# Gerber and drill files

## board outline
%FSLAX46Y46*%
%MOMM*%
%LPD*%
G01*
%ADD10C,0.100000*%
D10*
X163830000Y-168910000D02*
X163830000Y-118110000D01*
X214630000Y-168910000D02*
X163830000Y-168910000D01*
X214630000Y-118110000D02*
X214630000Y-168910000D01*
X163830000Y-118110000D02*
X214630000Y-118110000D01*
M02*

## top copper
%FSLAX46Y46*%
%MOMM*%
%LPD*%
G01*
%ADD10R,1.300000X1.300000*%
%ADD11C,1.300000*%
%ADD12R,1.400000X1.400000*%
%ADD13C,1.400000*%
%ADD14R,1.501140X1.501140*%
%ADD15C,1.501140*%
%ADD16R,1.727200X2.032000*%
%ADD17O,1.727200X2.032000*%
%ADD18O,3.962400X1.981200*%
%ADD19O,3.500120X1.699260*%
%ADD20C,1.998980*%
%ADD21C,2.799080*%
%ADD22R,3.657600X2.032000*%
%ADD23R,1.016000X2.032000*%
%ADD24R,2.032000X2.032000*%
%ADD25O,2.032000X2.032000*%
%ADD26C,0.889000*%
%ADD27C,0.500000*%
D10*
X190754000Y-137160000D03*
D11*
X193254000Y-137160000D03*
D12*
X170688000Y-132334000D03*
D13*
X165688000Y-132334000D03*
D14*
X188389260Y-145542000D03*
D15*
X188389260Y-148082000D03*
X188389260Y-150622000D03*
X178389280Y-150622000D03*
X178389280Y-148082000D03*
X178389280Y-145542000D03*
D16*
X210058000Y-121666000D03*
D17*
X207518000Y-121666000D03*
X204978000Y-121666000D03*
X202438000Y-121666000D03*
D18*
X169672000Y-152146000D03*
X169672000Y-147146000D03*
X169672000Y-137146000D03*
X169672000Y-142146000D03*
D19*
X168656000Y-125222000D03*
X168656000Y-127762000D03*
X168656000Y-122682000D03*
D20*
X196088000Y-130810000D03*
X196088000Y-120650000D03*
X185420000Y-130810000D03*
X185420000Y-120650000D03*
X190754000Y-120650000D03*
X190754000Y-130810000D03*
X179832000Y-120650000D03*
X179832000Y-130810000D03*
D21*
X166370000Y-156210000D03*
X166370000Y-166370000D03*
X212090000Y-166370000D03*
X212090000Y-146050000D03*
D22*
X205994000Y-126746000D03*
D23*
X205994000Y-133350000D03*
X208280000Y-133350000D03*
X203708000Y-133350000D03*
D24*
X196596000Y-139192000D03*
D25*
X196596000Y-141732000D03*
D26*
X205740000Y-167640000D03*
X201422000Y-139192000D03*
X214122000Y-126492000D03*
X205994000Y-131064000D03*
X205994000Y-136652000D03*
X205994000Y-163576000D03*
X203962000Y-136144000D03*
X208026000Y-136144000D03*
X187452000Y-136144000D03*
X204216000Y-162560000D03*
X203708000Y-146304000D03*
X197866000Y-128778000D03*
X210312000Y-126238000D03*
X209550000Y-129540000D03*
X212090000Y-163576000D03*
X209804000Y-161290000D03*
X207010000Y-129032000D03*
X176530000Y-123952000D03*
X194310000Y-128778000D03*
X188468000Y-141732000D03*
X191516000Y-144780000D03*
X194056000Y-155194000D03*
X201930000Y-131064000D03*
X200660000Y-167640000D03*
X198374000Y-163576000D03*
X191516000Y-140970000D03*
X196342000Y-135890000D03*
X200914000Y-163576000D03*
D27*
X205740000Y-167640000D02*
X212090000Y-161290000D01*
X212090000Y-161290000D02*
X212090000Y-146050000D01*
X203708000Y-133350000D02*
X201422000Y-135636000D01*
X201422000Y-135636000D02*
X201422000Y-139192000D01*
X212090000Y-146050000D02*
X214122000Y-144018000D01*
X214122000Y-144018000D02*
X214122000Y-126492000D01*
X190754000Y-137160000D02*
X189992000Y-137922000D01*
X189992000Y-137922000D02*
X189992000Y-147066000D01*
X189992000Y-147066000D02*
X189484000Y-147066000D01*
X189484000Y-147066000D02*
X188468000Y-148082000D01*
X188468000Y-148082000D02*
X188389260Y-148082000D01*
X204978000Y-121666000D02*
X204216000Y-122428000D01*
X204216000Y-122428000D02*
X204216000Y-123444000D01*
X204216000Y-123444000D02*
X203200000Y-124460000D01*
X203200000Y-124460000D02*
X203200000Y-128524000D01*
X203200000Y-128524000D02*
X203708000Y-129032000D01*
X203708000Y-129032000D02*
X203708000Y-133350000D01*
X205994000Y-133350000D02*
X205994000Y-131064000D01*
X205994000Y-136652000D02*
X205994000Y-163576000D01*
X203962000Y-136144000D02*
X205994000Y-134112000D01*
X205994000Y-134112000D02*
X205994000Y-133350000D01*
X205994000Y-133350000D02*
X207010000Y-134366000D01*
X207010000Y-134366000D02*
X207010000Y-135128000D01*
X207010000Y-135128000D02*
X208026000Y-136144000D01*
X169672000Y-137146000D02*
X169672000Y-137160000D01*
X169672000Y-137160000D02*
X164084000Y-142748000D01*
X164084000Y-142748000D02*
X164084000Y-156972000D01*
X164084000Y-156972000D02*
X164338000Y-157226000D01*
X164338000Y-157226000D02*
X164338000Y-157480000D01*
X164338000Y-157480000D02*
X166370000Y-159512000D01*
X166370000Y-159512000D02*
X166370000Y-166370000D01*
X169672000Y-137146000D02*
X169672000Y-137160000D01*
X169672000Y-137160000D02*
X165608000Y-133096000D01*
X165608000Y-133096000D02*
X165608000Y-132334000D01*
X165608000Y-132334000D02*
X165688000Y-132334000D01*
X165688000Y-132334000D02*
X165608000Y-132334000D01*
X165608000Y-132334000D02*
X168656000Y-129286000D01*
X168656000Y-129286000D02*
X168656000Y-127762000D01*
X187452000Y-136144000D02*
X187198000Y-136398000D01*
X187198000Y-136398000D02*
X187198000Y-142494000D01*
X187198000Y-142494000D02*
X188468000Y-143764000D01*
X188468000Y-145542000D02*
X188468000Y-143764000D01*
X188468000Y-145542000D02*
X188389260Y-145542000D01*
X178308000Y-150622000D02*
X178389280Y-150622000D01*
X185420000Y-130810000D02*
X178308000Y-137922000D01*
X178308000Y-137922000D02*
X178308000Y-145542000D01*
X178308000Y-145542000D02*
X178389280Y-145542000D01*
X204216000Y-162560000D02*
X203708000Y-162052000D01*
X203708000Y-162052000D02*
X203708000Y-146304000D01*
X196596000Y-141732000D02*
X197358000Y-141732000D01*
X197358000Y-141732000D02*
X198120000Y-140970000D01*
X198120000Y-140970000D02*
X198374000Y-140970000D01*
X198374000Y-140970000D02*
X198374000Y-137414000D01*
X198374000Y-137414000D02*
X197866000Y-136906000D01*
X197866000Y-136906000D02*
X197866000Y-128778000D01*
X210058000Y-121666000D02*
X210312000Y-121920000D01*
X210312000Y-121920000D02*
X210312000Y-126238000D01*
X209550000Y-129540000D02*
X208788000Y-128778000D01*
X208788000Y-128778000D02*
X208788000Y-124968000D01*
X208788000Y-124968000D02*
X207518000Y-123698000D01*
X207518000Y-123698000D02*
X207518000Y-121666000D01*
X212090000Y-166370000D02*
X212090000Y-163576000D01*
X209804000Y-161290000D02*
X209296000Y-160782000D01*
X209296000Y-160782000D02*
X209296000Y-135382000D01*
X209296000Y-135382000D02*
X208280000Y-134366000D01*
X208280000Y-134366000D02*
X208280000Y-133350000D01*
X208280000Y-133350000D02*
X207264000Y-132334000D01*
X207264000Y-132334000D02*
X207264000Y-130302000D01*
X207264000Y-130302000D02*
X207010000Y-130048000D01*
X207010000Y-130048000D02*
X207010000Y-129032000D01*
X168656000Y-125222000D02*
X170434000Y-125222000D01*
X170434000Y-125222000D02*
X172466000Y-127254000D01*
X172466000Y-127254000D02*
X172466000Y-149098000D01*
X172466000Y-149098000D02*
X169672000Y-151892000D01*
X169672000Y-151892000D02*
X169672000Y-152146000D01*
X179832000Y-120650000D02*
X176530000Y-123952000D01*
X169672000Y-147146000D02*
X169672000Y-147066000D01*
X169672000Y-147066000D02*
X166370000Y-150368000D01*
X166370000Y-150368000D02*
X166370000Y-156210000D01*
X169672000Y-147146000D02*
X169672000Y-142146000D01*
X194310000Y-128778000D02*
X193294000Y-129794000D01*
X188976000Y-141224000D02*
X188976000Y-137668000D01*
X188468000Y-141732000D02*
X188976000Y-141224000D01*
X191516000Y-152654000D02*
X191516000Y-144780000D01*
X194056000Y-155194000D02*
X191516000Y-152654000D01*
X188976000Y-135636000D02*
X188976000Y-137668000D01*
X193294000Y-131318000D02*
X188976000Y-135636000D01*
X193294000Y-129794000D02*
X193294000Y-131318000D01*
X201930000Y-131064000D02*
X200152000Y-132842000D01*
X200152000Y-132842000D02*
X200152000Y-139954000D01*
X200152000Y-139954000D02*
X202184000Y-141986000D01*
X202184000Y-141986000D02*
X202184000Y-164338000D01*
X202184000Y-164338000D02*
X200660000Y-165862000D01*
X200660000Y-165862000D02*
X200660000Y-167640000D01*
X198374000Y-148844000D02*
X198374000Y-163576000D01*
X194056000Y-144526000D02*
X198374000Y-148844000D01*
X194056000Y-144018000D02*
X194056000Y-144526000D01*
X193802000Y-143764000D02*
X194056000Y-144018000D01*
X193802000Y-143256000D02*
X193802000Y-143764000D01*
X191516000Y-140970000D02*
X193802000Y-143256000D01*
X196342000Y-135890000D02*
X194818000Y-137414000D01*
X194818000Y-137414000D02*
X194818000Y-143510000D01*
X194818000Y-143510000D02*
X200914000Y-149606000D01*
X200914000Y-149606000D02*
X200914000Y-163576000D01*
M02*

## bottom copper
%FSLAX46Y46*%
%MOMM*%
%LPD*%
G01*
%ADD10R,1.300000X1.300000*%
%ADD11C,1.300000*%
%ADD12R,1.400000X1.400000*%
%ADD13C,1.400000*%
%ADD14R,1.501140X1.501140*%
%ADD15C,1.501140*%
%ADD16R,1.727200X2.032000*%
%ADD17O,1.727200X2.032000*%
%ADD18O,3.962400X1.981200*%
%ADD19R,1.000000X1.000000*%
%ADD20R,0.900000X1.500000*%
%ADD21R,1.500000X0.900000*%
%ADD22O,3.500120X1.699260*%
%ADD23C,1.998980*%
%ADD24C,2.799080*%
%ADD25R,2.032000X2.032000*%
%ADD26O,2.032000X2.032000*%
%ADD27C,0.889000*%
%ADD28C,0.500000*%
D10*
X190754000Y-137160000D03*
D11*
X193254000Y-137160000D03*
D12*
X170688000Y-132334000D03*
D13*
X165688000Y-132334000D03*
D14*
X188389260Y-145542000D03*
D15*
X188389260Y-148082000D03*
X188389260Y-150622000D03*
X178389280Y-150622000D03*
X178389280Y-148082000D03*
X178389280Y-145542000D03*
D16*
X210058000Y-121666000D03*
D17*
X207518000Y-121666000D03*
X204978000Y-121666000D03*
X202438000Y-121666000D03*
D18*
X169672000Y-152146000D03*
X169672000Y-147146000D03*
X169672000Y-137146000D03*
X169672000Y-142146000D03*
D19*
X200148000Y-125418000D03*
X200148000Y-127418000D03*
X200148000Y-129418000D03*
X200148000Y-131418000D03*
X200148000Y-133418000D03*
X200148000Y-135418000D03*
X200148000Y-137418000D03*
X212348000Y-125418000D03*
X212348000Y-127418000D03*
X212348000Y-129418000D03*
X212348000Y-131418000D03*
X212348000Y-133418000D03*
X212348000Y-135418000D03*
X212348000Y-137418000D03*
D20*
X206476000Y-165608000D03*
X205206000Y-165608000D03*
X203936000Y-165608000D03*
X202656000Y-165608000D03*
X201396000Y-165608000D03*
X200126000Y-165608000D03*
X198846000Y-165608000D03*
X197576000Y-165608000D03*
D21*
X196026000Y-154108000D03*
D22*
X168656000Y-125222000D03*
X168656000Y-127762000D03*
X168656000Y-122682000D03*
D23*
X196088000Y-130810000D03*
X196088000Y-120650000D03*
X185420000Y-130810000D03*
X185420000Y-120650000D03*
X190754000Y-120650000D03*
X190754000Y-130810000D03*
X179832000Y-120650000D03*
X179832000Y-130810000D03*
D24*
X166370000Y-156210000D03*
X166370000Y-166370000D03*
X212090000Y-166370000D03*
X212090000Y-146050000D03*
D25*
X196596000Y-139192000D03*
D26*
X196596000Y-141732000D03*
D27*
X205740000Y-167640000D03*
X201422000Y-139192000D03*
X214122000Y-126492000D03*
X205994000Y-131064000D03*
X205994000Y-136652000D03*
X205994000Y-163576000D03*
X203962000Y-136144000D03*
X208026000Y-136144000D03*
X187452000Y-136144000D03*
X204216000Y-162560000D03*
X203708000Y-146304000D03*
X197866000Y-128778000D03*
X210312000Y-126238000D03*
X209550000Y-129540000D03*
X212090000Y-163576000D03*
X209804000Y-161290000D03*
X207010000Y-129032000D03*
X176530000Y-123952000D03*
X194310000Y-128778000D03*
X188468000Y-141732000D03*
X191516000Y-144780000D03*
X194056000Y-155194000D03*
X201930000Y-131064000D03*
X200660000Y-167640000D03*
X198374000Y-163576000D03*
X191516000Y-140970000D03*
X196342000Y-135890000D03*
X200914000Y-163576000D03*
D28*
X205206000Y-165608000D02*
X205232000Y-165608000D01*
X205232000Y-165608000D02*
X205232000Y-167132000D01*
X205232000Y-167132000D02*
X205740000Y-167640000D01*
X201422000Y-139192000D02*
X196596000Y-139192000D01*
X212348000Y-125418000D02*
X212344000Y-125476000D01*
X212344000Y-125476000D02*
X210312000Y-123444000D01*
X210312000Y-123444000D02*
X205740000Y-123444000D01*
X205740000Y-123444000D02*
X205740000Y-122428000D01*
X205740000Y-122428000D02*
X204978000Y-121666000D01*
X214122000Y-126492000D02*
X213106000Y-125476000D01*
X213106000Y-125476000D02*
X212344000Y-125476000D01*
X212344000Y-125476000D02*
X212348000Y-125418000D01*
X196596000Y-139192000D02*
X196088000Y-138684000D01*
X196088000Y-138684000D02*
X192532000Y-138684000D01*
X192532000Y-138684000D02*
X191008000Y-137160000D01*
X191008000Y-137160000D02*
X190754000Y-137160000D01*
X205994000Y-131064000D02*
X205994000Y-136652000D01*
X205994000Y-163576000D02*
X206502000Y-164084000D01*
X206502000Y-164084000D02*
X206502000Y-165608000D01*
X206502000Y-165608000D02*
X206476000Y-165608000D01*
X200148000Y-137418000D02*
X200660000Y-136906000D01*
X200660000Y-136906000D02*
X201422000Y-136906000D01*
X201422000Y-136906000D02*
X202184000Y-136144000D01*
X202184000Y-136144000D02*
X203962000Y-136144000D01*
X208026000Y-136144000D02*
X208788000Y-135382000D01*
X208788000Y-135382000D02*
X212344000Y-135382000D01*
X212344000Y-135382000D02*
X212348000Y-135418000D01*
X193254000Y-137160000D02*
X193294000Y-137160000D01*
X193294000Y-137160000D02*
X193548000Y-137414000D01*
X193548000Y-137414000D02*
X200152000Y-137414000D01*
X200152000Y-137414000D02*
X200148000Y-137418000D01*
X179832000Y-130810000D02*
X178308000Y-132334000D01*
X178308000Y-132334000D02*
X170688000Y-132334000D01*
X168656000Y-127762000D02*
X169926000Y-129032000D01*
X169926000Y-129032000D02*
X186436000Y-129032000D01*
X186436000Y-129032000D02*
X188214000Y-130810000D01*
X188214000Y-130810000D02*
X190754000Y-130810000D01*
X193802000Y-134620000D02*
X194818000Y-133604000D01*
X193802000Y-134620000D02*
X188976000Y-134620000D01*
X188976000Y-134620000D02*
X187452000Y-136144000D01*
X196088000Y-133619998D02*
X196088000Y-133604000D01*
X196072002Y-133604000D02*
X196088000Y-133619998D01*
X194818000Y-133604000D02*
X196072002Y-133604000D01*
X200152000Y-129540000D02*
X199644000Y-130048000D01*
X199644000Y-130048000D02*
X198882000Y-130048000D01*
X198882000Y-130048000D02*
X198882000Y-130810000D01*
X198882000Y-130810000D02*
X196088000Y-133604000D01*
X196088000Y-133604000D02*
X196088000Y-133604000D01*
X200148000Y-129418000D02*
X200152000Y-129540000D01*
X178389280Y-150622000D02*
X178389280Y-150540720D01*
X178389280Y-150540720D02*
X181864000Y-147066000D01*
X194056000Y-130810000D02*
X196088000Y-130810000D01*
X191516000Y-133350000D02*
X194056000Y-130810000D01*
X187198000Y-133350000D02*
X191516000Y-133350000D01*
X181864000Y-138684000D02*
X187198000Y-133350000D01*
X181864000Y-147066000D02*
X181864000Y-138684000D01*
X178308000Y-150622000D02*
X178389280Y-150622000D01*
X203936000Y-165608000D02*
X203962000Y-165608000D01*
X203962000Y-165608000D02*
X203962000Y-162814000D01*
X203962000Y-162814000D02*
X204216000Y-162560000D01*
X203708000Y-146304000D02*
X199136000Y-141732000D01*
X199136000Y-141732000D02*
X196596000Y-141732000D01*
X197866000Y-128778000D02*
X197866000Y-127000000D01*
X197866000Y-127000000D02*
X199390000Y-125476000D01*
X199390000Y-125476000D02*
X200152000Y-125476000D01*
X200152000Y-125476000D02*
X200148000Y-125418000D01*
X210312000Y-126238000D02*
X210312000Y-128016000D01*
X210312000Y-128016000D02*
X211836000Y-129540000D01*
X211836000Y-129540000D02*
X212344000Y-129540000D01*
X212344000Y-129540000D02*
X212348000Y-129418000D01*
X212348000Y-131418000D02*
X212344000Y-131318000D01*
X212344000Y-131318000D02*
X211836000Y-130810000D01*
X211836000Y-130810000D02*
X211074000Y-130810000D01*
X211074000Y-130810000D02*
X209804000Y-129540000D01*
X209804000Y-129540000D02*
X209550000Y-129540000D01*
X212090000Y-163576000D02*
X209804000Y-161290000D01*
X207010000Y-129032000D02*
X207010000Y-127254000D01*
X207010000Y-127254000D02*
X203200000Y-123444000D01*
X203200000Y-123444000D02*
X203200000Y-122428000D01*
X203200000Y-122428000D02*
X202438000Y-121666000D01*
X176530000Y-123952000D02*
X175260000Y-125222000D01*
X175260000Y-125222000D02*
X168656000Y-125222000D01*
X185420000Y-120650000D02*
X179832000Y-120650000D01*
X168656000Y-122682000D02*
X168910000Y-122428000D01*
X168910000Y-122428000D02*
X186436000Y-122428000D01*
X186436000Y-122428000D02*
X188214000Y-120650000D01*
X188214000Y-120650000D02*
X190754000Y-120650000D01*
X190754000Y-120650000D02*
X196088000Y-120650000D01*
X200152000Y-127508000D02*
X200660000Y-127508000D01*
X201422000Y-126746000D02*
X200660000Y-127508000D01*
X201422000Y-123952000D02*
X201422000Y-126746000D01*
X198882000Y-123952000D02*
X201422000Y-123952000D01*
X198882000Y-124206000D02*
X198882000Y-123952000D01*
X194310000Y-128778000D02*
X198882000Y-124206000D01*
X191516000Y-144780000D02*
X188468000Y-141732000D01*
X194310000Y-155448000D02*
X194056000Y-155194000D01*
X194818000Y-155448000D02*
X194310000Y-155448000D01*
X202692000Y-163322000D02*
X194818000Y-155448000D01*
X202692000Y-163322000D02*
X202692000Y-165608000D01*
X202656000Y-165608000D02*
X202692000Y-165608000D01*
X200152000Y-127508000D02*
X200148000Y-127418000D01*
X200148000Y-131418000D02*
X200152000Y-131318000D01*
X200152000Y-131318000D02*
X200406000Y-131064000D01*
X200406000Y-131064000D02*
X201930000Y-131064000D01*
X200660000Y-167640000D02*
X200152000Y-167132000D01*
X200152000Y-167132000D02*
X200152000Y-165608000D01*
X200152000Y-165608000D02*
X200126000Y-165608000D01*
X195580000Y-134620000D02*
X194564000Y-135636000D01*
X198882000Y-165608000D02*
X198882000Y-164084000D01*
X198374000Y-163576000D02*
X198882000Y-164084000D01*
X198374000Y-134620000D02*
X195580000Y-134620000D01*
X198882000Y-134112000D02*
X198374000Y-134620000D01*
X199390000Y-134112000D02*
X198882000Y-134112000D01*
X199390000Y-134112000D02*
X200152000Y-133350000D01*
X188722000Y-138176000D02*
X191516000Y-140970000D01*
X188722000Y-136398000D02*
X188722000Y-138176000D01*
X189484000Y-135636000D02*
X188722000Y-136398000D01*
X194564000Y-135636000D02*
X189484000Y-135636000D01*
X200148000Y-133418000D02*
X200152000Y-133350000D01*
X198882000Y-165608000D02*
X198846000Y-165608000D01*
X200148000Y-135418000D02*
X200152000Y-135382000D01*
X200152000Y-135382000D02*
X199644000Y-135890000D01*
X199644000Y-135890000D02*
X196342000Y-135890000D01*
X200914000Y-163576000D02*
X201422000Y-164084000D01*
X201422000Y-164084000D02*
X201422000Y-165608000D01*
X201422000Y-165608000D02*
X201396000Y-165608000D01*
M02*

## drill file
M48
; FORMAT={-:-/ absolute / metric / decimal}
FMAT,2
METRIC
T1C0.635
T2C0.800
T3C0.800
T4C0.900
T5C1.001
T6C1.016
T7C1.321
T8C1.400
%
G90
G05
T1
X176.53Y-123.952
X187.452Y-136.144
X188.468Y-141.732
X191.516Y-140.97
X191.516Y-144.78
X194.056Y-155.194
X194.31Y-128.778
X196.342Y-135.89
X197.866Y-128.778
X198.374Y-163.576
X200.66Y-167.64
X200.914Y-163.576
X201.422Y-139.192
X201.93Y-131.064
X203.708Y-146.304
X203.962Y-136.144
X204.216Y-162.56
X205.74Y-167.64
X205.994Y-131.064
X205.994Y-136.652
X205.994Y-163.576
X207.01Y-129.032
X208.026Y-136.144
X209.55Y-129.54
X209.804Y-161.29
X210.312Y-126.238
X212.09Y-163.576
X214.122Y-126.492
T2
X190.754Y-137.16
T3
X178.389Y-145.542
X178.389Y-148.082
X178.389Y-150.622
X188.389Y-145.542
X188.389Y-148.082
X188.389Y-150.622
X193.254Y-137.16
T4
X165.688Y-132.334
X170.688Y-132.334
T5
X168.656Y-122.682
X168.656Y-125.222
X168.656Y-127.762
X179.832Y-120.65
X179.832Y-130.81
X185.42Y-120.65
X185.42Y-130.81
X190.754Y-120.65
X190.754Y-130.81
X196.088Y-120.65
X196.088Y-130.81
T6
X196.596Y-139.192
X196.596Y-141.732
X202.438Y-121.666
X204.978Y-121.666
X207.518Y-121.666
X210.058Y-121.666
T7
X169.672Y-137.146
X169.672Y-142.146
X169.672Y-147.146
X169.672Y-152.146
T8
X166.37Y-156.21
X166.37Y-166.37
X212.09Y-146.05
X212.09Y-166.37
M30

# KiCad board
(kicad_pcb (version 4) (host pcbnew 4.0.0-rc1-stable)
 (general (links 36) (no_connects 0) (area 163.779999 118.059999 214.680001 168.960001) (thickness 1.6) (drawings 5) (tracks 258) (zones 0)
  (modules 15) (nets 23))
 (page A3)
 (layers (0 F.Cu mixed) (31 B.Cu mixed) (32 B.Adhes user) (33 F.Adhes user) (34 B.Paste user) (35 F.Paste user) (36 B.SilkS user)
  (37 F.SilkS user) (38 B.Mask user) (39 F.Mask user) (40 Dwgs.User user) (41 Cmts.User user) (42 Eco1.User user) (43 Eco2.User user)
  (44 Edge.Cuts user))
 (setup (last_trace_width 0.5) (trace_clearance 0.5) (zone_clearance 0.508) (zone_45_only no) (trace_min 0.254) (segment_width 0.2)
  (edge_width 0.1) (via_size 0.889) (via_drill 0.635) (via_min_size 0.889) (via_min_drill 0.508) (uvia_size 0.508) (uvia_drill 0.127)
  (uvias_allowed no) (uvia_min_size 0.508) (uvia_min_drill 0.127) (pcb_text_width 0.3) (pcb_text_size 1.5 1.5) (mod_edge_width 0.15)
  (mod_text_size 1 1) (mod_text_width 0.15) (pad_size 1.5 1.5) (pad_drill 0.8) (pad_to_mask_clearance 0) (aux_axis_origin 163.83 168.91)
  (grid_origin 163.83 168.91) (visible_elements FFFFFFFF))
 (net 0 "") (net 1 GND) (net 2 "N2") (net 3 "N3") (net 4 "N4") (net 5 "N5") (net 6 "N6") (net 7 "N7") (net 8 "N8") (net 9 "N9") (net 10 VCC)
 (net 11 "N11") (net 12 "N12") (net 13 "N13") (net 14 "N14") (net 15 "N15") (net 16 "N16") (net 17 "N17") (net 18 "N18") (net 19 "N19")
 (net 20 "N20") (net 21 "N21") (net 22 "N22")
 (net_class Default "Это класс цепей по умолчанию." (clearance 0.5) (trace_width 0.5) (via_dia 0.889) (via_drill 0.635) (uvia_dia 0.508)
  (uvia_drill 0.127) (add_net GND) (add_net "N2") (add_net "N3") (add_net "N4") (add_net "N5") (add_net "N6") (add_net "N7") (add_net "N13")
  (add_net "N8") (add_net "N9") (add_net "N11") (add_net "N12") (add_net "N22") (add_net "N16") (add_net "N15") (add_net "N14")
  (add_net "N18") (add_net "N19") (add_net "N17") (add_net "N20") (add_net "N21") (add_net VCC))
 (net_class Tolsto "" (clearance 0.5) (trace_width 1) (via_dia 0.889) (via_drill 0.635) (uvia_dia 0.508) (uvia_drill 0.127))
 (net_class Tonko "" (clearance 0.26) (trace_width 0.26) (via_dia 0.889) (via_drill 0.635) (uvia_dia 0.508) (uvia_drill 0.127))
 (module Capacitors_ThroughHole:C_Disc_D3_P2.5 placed (layer B.Cu) (at 190.754 137.16)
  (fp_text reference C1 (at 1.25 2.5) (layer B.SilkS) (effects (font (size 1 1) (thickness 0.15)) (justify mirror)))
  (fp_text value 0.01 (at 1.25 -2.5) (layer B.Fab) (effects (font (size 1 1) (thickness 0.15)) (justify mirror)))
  (pad 1 thru_hole rect (at 0 0) (size 1.3 1.3) (drill 0.8) (layers *.Cu *.Mask B.SilkS) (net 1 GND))
  (pad 2 thru_hole circle (at 2.5 0) (size 1.3 1.3) (drill 0.8001) (layers *.Cu *.Mask B.SilkS) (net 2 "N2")))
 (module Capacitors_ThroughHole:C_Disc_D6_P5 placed (layer F.Cu) (at 170.688 132.334 180)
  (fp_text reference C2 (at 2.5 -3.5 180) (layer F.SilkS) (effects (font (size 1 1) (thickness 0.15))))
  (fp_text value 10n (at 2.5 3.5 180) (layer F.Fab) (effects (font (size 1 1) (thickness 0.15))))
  (pad 1 thru_hole rect (at 0 0 180) (size 1.4 1.4) (drill 0.9) (layers *.Cu *.Mask F.SilkS) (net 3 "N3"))
  (pad 2 thru_hole circle (at 5 0 180) (size 1.4 1.4) (drill 0.9) (layers *.Cu *.Mask F.SilkS) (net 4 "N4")))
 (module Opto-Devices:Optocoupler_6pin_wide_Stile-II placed (layer B.Cu) (at 183.388 148.082 270)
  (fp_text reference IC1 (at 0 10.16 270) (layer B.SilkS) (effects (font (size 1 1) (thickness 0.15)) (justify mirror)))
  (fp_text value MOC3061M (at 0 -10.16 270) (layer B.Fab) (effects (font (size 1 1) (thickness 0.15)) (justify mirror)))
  (pad 1 thru_hole rect (at -2.54 -5.00126 270) (size 1.50114 1.50114) (drill 0.8001) (layers *.Cu *.Mask B.SilkS) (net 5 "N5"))
  (pad 2 thru_hole circle (at 0 -5.00126 270) (size 1.50114 1.50114) (drill 0.8001) (layers *.Cu *.Mask B.SilkS) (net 1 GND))
  (pad 3 thru_hole circle (at 2.54 -5.00126 270) (size 1.50114 1.50114) (drill 0.8001) (layers *.Cu *.Mask B.SilkS))
  (pad 4 thru_hole circle (at 2.54 4.99872 270) (size 1.50114 1.50114) (drill 0.8001) (layers *.Cu *.Mask B.SilkS) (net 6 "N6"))
  (pad 5 thru_hole circle (at 0 4.99872 270) (size 1.50114 1.50114) (drill 0.8001) (layers *.Cu *.Mask B.SilkS))
  (pad 6 thru_hole circle (at -2.54 4.99872 270) (size 1.50114 1.50114) (drill 0.8001) (layers *.Cu *.Mask B.SilkS) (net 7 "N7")))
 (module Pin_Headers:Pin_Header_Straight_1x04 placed (layer F.Cu) (at 210.058 121.666 270)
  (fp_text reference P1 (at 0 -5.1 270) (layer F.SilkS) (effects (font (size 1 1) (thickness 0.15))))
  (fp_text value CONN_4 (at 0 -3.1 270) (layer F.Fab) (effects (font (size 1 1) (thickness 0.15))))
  (pad 1 thru_hole rect (at 0 0 270) (size 2.032 1.7272) (drill 1.016) (layers *.Cu *.Mask F.SilkS) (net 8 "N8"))
  (pad 2 thru_hole oval (at 0 2.54 270) (size 2.032 1.7272) (drill 1.016) (layers *.Cu *.Mask F.SilkS) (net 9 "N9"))
  (pad 3 thru_hole oval (at 0 5.08 270) (size 2.032 1.7272) (drill 1.016) (layers *.Cu *.Mask F.SilkS) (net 1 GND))
  (pad 4 thru_hole oval (at 0 7.62 270) (size 2.032 1.7272) (drill 1.016) (layers *.Cu *.Mask F.SilkS) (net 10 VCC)))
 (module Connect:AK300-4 (layer B.Cu) (at 169.672 152.146 90)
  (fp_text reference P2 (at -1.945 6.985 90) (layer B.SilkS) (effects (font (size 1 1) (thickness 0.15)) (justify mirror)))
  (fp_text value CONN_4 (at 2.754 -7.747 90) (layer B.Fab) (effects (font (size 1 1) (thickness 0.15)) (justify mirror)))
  (pad 1 thru_hole oval (at 0 0 90) (size 1.9812 3.9624) (drill 1.3208) (layers *.Cu B.Paste B.SilkS B.Mask) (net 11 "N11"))
  (pad 2 thru_hole oval (at 5 0 90) (size 1.9812 3.9624) (drill 1.3208) (layers *.Cu B.Paste B.SilkS B.Mask) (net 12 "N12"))
  (pad 4 thru_hole oval (at 15 0 90) (size 1.9812 3.9624) (drill 1.3208) (layers *.Cu B.Paste B.SilkS B.Mask) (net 4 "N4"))
  (pad 3 thru_hole oval (at 10 0 90) (size 1.9812 3.9624) (drill 1.3208) (layers *.Cu *.Mask B.SilkS) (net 12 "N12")))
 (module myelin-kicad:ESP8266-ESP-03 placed (layer B.Cu) (at 206.248 131.318)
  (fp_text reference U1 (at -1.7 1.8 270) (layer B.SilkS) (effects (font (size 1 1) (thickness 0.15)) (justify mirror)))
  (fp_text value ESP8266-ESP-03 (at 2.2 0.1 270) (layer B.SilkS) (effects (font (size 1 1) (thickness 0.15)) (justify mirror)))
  (pad 14 smd rect (at -6.1 -5.9) (size 1 1) (layers B.Cu B.Paste B.Mask) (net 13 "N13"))
  (pad 13 smd rect (at -6.1 -3.9) (size 1 1) (layers B.Cu B.Paste B.Mask) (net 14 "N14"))
  (pad 12 smd rect (at -6.1 -1.9) (size 1 1) (layers B.Cu B.Paste B.Mask) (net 5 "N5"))
  (pad 11 smd rect (at -6.1 0.1) (size 1 1) (layers B.Cu B.Paste B.Mask) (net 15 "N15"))
  (pad 10 smd rect (at -6.1 2.1) (size 1 1) (layers B.Cu B.Paste B.Mask) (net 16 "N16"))
  (pad 9 smd rect (at -6.1 4.1) (size 1 1) (layers B.Cu B.Paste B.Mask) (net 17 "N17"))
  (pad 8 smd rect (at -6.1 6.1) (size 1 1) (layers B.Cu B.Paste B.Mask) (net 2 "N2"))
  (pad 1 smd rect (at 6.1 -5.9) (size 1 1) (layers B.Cu B.Paste B.Mask) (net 1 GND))
  (pad 2 smd rect (at 6.1 -3.9) (size 1 1) (layers B.Cu B.Paste B.Mask))
  (pad 3 smd rect (at 6.1 -1.9) (size 1 1) (layers B.Cu B.Paste B.Mask) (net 8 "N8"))
  (pad 4 smd rect (at 6.1 0.1) (size 1 1) (layers B.Cu B.Paste B.Mask) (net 9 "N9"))
  (pad 5 smd rect (at 6.1 2.1) (size 1 1) (layers B.Cu B.Paste B.Mask) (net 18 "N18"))
  (pad 6 smd rect (at 6.1 4.1) (size 1 1) (layers B.Cu B.Paste B.Mask) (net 2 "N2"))
  (pad 7 smd rect (at 6.1 6.1) (size 1 1) (layers B.Cu B.Paste B.Mask) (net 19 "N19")))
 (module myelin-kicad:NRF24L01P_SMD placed (layer B.Cu) (at 208.026 165.608 90)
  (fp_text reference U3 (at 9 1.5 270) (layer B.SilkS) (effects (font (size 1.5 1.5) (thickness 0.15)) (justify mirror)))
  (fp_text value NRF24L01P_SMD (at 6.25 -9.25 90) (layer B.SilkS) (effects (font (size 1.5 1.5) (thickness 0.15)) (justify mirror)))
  (pad 1 smd rect (at 0 -1.55 90) (size 1.5 0.9) (layers B.Cu B.Paste B.Mask) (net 2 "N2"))
  (pad 2 smd rect (at 0 -2.82 90) (size 1.5 0.9) (layers B.Cu B.Paste B.Mask) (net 1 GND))
  (pad 3 smd rect (at 0 -4.09 90) (size 1.5 0.9) (layers B.Cu B.Paste B.Mask) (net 13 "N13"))
  (pad 4 smd rect (at 0 -5.37 90) (size 1.5 0.9) (layers B.Cu B.Paste B.Mask) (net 14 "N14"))
  (pad 5 smd rect (at 0 -6.63 90) (size 1.5 0.9) (layers B.Cu B.Paste B.Mask) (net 17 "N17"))
  (pad 6 smd rect (at 0 -7.9 90) (size 1.5 0.9) (layers B.Cu B.Paste B.Mask) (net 15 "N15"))
  (pad 7 smd rect (at 0 -9.18 90) (size 1.5 0.9) (layers B.Cu B.Paste B.Mask) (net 16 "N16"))
  (pad 8 smd rect (at 0 -10.45 90) (size 1.5 0.9) (layers B.Cu B.Paste B.Mask) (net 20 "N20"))
  (pad 9 smd rect (at 11.5 -12 90) (size 0.9 1.5) (layers B.Cu B.Paste B.Mask) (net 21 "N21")))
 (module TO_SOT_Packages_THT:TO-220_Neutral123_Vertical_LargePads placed (layer F.Cu) (at 168.656 125.222 90)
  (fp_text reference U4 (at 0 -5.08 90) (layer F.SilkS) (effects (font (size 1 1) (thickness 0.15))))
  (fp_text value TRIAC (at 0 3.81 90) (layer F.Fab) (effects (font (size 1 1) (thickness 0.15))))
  (pad 2 thru_hole oval (at 0 0 180) (size 3.50012 1.69926) (drill 1.00076) (layers *.Cu *.Mask F.SilkS) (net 11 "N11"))
  (pad 1 thru_hole oval (at -2.54 0 180) (size 3.50012 1.69926) (drill 1.00076) (layers *.Cu *.Mask F.SilkS) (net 4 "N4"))
  (pad 3 thru_hole oval (at 2.54 0 180) (size 3.50012 1.69926) (drill 1.00076) (layers *.Cu *.Mask F.SilkS) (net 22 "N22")))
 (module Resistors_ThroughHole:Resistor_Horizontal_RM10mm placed (layer F.Cu) (at 196.088 125.73 90)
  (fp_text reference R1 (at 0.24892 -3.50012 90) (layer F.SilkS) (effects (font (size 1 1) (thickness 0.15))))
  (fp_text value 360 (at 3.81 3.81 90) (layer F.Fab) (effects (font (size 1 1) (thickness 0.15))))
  (pad 1 thru_hole circle (at -5.08 0 90) (size 1.99898 1.99898) (drill 1.00076) (layers *.Cu *.SilkS *.Mask) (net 6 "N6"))
  (pad 2 thru_hole circle (at 5.08 0 90) (size 1.99898 1.99898) (drill 1.00076) (layers *.Cu *.SilkS *.Mask) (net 22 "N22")))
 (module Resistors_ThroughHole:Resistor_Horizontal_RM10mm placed (layer F.Cu) (at 185.42 125.73 90)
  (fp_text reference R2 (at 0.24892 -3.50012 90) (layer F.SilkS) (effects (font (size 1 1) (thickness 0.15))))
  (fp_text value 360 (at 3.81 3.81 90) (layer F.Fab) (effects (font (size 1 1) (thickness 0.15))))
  (pad 1 thru_hole circle (at -5.08 0 90) (size 1.99898 1.99898) (drill 1.00076) (layers *.Cu *.SilkS *.Mask) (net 7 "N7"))
  (pad 2 thru_hole circle (at 5.08 0 90) (size 1.99898 1.99898) (drill 1.00076) (layers *.Cu *.SilkS *.Mask) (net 11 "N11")))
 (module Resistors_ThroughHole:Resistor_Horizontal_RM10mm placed (layer F.Cu) (at 190.754 125.73 270)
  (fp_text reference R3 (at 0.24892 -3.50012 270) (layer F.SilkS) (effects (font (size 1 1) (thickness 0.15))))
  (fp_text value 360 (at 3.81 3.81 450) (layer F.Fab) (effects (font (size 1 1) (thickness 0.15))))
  (pad 1 thru_hole circle (at -5.08 0 270) (size 1.99898 1.99898) (drill 1.00076) (layers *.Cu *.SilkS *.Mask) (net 22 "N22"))
  (pad 2 thru_hole circle (at 5.08 0 270) (size 1.99898 1.99898) (drill 1.00076) (layers *.Cu *.SilkS *.Mask) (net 4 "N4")))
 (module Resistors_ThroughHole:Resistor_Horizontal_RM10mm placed (layer F.Cu) (at 179.832 125.73 270)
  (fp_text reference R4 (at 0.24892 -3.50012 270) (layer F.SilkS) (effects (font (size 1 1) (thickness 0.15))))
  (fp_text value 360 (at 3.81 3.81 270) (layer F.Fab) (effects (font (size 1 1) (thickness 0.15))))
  (pad 1 thru_hole circle (at -5.08 0 270) (size 1.99898 1.99898) (drill 1.00076) (layers *.Cu *.SilkS *.Mask) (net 11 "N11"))
  (pad 2 thru_hole circle (at 5.08 0 270) (size 1.99898 1.99898) (drill 1.00076) (layers *.Cu *.SilkS *.Mask) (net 3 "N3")))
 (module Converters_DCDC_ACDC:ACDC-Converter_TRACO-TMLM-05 (layer F.Cu) (at 166.37 156.21)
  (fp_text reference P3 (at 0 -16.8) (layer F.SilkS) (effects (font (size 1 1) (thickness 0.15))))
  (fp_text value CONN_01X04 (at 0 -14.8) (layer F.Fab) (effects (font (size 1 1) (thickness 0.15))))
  (pad 1 thru_hole circle (at 0 0) (size 2.79908 2.79908) (drill 1.39954) (layers *.Cu *.Mask F.SilkS) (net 12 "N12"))
  (pad 2 thru_hole circle (at 0 10.16) (size 2.79908 2.79908) (drill 1.39954) (layers *.Cu *.Mask F.SilkS) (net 4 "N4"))
  (pad 3 thru_hole circle (at 45.72 10.16) (size 2.79908 2.79908) (drill 1.39954) (layers *.Cu *.Mask F.SilkS) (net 10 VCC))
  (pad 4 thru_hole circle (at 45.72 -10.16) (size 2.79908 2.79908) (drill 1.39954) (layers *.Cu *.Mask F.SilkS) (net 1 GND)))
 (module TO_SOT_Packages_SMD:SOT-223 (layer F.Cu) (at 205.994 130.048)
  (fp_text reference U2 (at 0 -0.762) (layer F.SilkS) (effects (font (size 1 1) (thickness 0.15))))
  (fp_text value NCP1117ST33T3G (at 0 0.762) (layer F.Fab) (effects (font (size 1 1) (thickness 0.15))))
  (pad 4 smd rect (at 0 -3.302) (size 3.6576 2.032) (layers F.Cu F.Paste F.Mask))
  (pad 2 smd rect (at 0 3.302) (size 1.016 2.032) (layers F.Cu F.Paste F.Mask) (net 2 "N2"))
  (pad 3 smd rect (at 2.286 3.302) (size 1.016 2.032) (layers F.Cu F.Paste F.Mask) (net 10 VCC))
  (pad 1 smd rect (at -2.286 3.302) (size 1.016 2.032) (layers F.Cu F.Paste F.Mask) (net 1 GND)))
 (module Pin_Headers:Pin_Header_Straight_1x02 (layer F.Cu) (at 196.596 139.192)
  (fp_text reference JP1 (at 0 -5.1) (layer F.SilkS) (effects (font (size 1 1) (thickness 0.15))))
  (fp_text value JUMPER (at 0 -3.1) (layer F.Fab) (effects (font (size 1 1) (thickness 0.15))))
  (pad 1 thru_hole rect (at 0 0) (size 2.032 2.032) (drill 1.016) (layers *.Cu *.Mask F.SilkS) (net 1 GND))
  (pad 2 thru_hole oval (at 0 2.54) (size 2.032 2.032) (drill 1.016) (layers *.Cu *.Mask F.SilkS) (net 13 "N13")))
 (gr_line (start 163.83 168.91) (end 163.83 118.11) (angle 90) (layer Edge.Cuts) (width 0.1))
 (gr_line (start 214.63 168.91) (end 163.83 168.91) (angle 90) (layer Edge.Cuts) (width 0.1))
 (gr_line (start 214.63 118.11) (end 214.63 168.91) (angle 90) (layer Edge.Cuts) (width 0.1))
 (gr_line (start 163.83 118.11) (end 214.63 118.11) (angle 90) (layer Edge.Cuts) (width 0.1))
 (segment (start 205.206 165.608) (end 205.232 165.608) (width 0.5) (layer B.Cu) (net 1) (status 80000))
 (segment (start 205.232 165.608) (end 205.232 167.132) (width 0.5) (layer B.Cu) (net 1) (status 80000))
 (segment (start 205.232 167.132) (end 205.74 167.64) (width 0.5) (layer B.Cu) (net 1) (status 80000))
 (via (at 205.74 167.64) (size 0.889) (layers F.Cu B.Cu) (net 1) (status 80000))
 (segment (start 205.74 167.64) (end 212.09 161.29) (width 0.5) (layer F.Cu) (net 1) (status 80000))
 (segment (start 212.09 161.29) (end 212.09 146.05) (width 0.5) (layer F.Cu) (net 1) (status 80000))
 (segment (start 203.708 133.35) (end 201.422 135.636) (width 0.5) (layer F.Cu) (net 1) (status 80000))
 (segment (start 201.422 135.636) (end 201.422 139.192) (width 0.5) (layer F.Cu) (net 1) (status 80000))
 (via (at 201.422 139.192) (size 0.889) (layers F.Cu B.Cu) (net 1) (status 80000))
 (segment (start 201.422 139.192) (end 196.596 139.192) (width 0.5) (layer B.Cu) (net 1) (status 80000))
 (segment (start 212.348 125.418) (end 212.344 125.476) (width 0.5) (layer B.Cu) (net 1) (status 80000))
 (segment (start 212.344 125.476) (end 210.312 123.444) (width 0.5) (layer B.Cu) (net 1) (status 80000))
 (segment (start 210.312 123.444) (end 205.74 123.444) (width 0.5) (layer B.Cu) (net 1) (status 80000))
 (segment (start 205.74 123.444) (end 205.74 122.428) (width 0.5) (layer B.Cu) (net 1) (status 80000))
 (segment (start 205.74 122.428) (end 204.978 121.666) (width 0.5) (layer B.Cu) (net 1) (status 80000))
 (segment (start 212.09 146.05) (end 214.122 144.018) (width 0.5) (layer F.Cu) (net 1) (status 80000))
 (segment (start 214.122 144.018) (end 214.122 126.492) (width 0.5) (layer F.Cu) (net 1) (status 80000))
 (via (at 214.122 126.492) (size 0.889) (layers F.Cu B.Cu) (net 1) (status 80000))
 (segment (start 214.122 126.492) (end 213.106 125.476) (width 0.5) (layer B.Cu) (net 1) (status 80000))
 (segment (start 213.106 125.476) (end 212.344 125.476) (width 0.5) (layer B.Cu) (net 1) (status 80000))
 (segment (start 212.344 125.476) (end 212.348 125.418) (width 0.5) (layer B.Cu) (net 1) (status 80000))
 (segment (start 190.754 137.16) (end 189.992 137.922) (width 0.5) (layer F.Cu) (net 1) (status 80000))
 (segment (start 189.992 137.922) (end 189.992 147.066) (width 0.5) (layer F.Cu) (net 1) (status 80000))
 (segment (start 189.992 147.066) (end 189.484 147.066) (width 0.5) (layer F.Cu) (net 1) (status 80000))
 (segment (start 189.484 147.066) (end 188.468 148.082) (width 0.5) (layer F.Cu) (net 1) (status 80000))
 (segment (start 188.468 148.082) (end 188.38926 148.082) (width 0.5) (layer F.Cu) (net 1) (status 80000))
 (segment (start 204.978 121.666) (end 204.216 122.428) (width 0.5) (layer F.Cu) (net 1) (status 80000))
 (segment (start 204.216 122.428) (end 204.216 123.444) (width 0.5) (layer F.Cu) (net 1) (status 80000))
 (segment (start 204.216 123.444) (end 203.2 124.46) (width 0.5) (layer F.Cu) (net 1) (status 80000))
 (segment (start 203.2 124.46) (end 203.2 128.524) (width 0.5) (layer F.Cu) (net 1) (status 80000))
 (segment (start 203.2 128.524) (end 203.708 129.032) (width 0.5) (layer F.Cu) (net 1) (status 80000))
 (segment (start 203.708 129.032) (end 203.708 133.35) (width 0.5) (layer F.Cu) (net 1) (status 80000))
 (segment (start 196.596 139.192) (end 196.088 138.684) (width 0.5) (layer B.Cu) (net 1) (status 80000))
 (segment (start 196.088 138.684) (end 192.532 138.684) (width 0.5) (layer B.Cu) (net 1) (status 80000))
 (segment (start 192.532 138.684) (end 191.008 137.16) (width 0.5) (layer B.Cu) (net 1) (status 80000))
 (segment (start 191.008 137.16) (end 190.754 137.16) (width 0.5) (layer B.Cu) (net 1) (status 80000))
 (segment (start 205.994 133.35) (end 205.994 131.064) (width 0.5) (layer F.Cu) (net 2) (status 80000))
 (via (at 205.994 131.064) (size 0.889) (layers F.Cu B.Cu) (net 2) (status 80000))
 (segment (start 205.994 131.064) (end 205.994 136.652) (width 0.5) (layer B.Cu) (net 2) (status 80000))
 (via (at 205.994 136.652) (size 0.889) (layers F.Cu B.Cu) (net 2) (status 80000))
 (segment (start 205.994 136.652) (end 205.994 163.576) (width 0.5) (layer F.Cu) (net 2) (status 80000))
 (via (at 205.994 163.576) (size 0.889) (layers F.Cu B.Cu) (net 2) (status 80000))
 (segment (start 205.994 163.576) (end 206.502 164.084) (width 0.5) (layer B.Cu) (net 2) (status 80000))
 (segment (start 206.502 164.084) (end 206.502 165.608) (width 0.5) (layer B.Cu) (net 2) (status 80000))
 (segment (start 206.502 165.608) (end 206.476 165.608) (width 0.5) (layer B.Cu) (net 2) (status 80000))
 (segment (start 200.148 137.418) (end 200.66 136.906) (width 0.5) (layer B.Cu) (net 2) (status 80000))
 (segment (start 200.66 136.906) (end 201.422 136.906) (width 0.5) (layer B.Cu) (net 2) (status 80000))
 (segment (start 201.422 136.906) (end 202.184 136.144) (width 0.5) (layer B.Cu) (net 2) (status 80000))
 (segment (start 202.184 136.144) (end 203.962 136.144) (width 0.5) (layer B.Cu) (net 2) (status 80000))
 (via (at 203.962 136.144) (size 0.889) (layers F.Cu B.Cu) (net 2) (status 80000))
 (segment (start 203.962 136.144) (end 205.994 134.112) (width 0.5) (layer F.Cu) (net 2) (status 80000))
 (segment (start 205.994 134.112) (end 205.994 133.35) (width 0.5) (layer F.Cu) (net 2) (status 80000))
 (segment (start 205.994 133.35) (end 207.01 134.366) (width 0.5) (layer F.Cu) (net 2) (status 80000))
 (segment (start 207.01 134.366) (end 207.01 135.128) (width 0.5) (layer F.Cu) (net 2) (status 80000))
 (segment (start 207.01 135.128) (end 208.026 136.144) (width 0.5) (layer F.Cu) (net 2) (status 80000))
 (via (at 208.026 136.144) (size 0.889) (layers F.Cu B.Cu) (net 2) (status 80000))
 (segment (start 208.026 136.144) (end 208.788 135.382) (width 0.5) (layer B.Cu) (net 2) (status 80000))
 (segment (start 208.788 135.382) (end 212.344 135.382) (width 0.5) (layer B.Cu) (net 2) (status 80000))
 (segment (start 212.344 135.382) (end 212.348 135.418) (width 0.5) (layer B.Cu) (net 2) (status 80000))
 (segment (start 193.254 137.16) (end 193.294 137.16) (width 0.5) (layer B.Cu) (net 2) (status 80000))
 (segment (start 193.294 137.16) (end 193.548 137.414) (width 0.5) (layer B.Cu) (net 2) (status 80000))
 (segment (start 193.548 137.414) (end 200.152 137.414) (width 0.5) (layer B.Cu) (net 2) (status 80000))
 (segment (start 200.152 137.414) (end 200.148 137.418) (width 0.5) (layer B.Cu) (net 2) (status 80000))
 (segment (start 179.832 130.81) (end 178.308 132.334) (width 0.5) (layer B.Cu) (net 3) (status 80000))
 (segment (start 178.308 132.334) (end 170.688 132.334) (width 0.5) (layer B.Cu) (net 3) (status 80000))
 (segment (start 169.672 137.146) (end 169.672 137.16) (width 0.5) (layer F.Cu) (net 4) (status 80000))
 (segment (start 169.672 137.16) (end 164.084 142.748) (width 0.5) (layer F.Cu) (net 4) (status 80000))
 (segment (start 164.084 142.748) (end 164.084 156.972) (width 0.5) (layer F.Cu) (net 4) (status 80000))
 (segment (start 164.084 156.972) (end 164.338 157.226) (width 0.5) (layer F.Cu) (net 4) (status 80000))
 (segment (start 164.338 157.226) (end 164.338 157.48) (width 0.5) (layer F.Cu) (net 4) (status 80000))
 (segment (start 164.338 157.48) (end 166.37 159.512) (width 0.5) (layer F.Cu) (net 4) (status 80000))
 (segment (start 166.37 159.512) (end 166.37 166.37) (width 0.5) (layer F.Cu) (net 4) (status 80000))
 (segment (start 168.656 127.762) (end 169.926 129.032) (width 0.5) (layer B.Cu) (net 4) (status 80000))
 (segment (start 169.926 129.032) (end 186.436 129.032) (width 0.5) (layer B.Cu) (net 4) (status 80000))
 (segment (start 186.436 129.032) (end 188.214 130.81) (width 0.5) (layer B.Cu) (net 4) (status 80000))
 (segment (start 188.214 130.81) (end 190.754 130.81) (width 0.5) (layer B.Cu) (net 4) (status 80000))
 (segment (start 169.672 137.146) (end 169.672 137.16) (width 0.5) (layer F.Cu) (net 4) (status 80000))
 (segment (start 169.672 137.16) (end 165.608 133.096) (width 0.5) (layer F.Cu) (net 4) (status 80000))
 (segment (start 165.608 133.096) (end 165.608 132.334) (width 0.5) (layer F.Cu) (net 4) (status 80000))
 (segment (start 165.608 132.334) (end 165.688 132.334) (width 0.5) (layer F.Cu) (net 4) (status 80000))
 (segment (start 165.688 132.334) (end 165.608 132.334) (width 0.5) (layer F.Cu) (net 4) (status 80000))
 (segment (start 165.608 132.334) (end 168.656 129.286) (width 0.5) (layer F.Cu) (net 4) (status 80000))
 (segment (start 168.656 129.286) (end 168.656 127.762) (width 0.5) (layer F.Cu) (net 4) (status 80000))
 (segment (start 193.802 134.62) (end 194.818 133.604) (width 0.5) (layer B.Cu) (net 5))
 (segment (start 193.802 134.62) (end 188.976 134.62) (width 0.5) (layer B.Cu) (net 5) (status 80000))
 (segment (start 188.976 134.62) (end 187.452 136.144) (width 0.5) (layer B.Cu) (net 5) (status 80000))
 (via (at 187.452 136.144) (size 0.889) (layers F.Cu B.Cu) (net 5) (status 80000))
 (segment (start 187.452 136.144) (end 187.198 136.398) (width 0.5) (layer F.Cu) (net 5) (status 80000))
 (segment (start 187.198 136.398) (end 187.198 142.494) (width 0.5) (layer F.Cu) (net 5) (status 80000))
 (segment (start 187.198 142.494) (end 188.468 143.764) (width 0.5) (layer F.Cu) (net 5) (status 80000))
 (segment (start 188.468 145.542) (end 188.468 143.764) (width 0.5) (layer F.Cu) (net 5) (status 80000))
 (segment (start 196.088 133.619998) (end 196.088 133.604) (width 0.5) (layer B.Cu) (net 5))
 (segment (start 196.072002 133.604) (end 196.088 133.619998) (width 0.5) (layer B.Cu) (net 5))
 (segment (start 194.818 133.604) (end 196.072002 133.604) (width 0.5) (layer B.Cu) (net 5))
 (segment (start 200.152 129.54) (end 199.644 130.048) (width 0.5) (layer B.Cu) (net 5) (status 80000))
 (segment (start 199.644 130.048) (end 198.882 130.048) (width 0.5) (layer B.Cu) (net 5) (status 80000))
 (segment (start 198.882 130.048) (end 198.882 130.81) (width 0.5) (layer B.Cu) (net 5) (status 80000))
 (segment (start 198.882 130.81) (end 196.088 133.604) (width 0.5) (layer B.Cu) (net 5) (status 80000))
 (segment (start 196.088 133.604) (end 196.088 133.604) (width 0.5) (layer B.Cu) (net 5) (status 80000))
 (segment (start 200.148 129.418) (end 200.152 129.54) (width 0.5) (layer B.Cu) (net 5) (status 80000))
 (segment (start 188.468 145.542) (end 188.38926 145.542) (width 0.5) (layer F.Cu) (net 5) (status 80000))
 (segment (start 178.38928 150.622) (end 178.38928 150.54072) (width 0.5) (layer B.Cu) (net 6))
 (segment (start 178.38928 150.54072) (end 181.864 147.066) (width 0.5) (layer B.Cu) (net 6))
 (segment (start 194.056 130.81) (end 196.088 130.81) (width 0.5) (layer B.Cu) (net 6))
 (segment (start 191.516 133.35) (end 194.056 130.81) (width 0.5) (layer B.Cu) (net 6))
 (segment (start 187.198 133.35) (end 191.516 133.35) (width 0.5) (layer B.Cu) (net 6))
 (segment (start 181.864 138.684) (end 187.198 133.35) (width 0.5) (layer B.Cu) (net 6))
 (segment (start 181.864 147.066) (end 181.864 138.684) (width 0.5) (layer B.Cu) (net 6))
 (segment (start 178.308 150.622) (end 178.38928 150.622) (width 0.5) (layer B.Cu) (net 6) (status 80000))
 (segment (start 178.308 150.622) (end 178.38928 150.622) (width 0.5) (layer F.Cu) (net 6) (status 80000))
 (segment (start 185.42 130.81) (end 178.308 137.922) (width 0.5) (layer F.Cu) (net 7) (status 80000))
 (segment (start 178.308 137.922) (end 178.308 145.542) (width 0.5) (layer F.Cu) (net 7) (status 80000))
 (segment (start 178.308 145.542) (end 178.38928 145.542) (width 0.5) (layer F.Cu) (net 7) (status 80000))
 (segment (start 203.936 165.608) (end 203.962 165.608) (width 0.5) (layer B.Cu) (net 13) (status 80000))
 (segment (start 203.962 165.608) (end 203.962 162.814) (width 0.5) (layer B.Cu) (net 13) (status 80000))
 (segment (start 203.962 162.814) (end 204.216 162.56) (width 0.5) (layer B.Cu) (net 13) (status 80000))
 (via (at 204.216 162.56) (size 0.889) (layers F.Cu B.Cu) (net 13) (status 80000))
 (segment (start 204.216 162.56) (end 203.708 162.052) (width 0.5) (layer F.Cu) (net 13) (status 80000))
 (segment (start 203.708 162.052) (end 203.708 146.304) (width 0.5) (layer F.Cu) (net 13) (status 80000))
 (via (at 203.708 146.304) (size 0.889) (layers F.Cu B.Cu) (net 13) (status 80000))
 (segment (start 203.708 146.304) (end 199.136 141.732) (width 0.5) (layer B.Cu) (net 13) (status 80000))
 (segment (start 199.136 141.732) (end 196.596 141.732) (width 0.5) (layer B.Cu) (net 13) (status 80000))
 (segment (start 196.596 141.732) (end 197.358 141.732) (width 0.5) (layer F.Cu) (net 13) (status 80000))
 (segment (start 197.358 141.732) (end 198.12 140.97) (width 0.5) (layer F.Cu) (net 13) (status 80000))
 (segment (start 198.12 140.97) (end 198.374 140.97) (width 0.5) (layer F.Cu) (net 13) (status 80000))
 (segment (start 198.374 140.97) (end 198.374 137.414) (width 0.5) (layer F.Cu) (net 13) (status 80000))
 (segment (start 198.374 137.414) (end 197.866 136.906) (width 0.5) (layer F.Cu) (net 13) (status 80000))
 (segment (start 197.866 136.906) (end 197.866 128.778) (width 0.5) (layer F.Cu) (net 13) (status 80000))
 (via (at 197.866 128.778) (size 0.889) (layers F.Cu B.Cu) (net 13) (status 80000))
 (segment (start 197.866 128.778) (end 197.866 127) (width 0.5) (layer B.Cu) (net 13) (status 80000))
 (segment (start 197.866 127) (end 199.39 125.476) (width 0.5) (layer B.Cu) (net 13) (status 80000))
 (segment (start 199.39 125.476) (end 200.152 125.476) (width 0.5) (layer B.Cu) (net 13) (status 80000))
 (segment (start 200.152 125.476) (end 200.148 125.418) (width 0.5) (layer B.Cu) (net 13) (status 80000))
 (segment (start 210.058 121.666) (end 210.312 121.92) (width 0.5) (layer F.Cu) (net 8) (status 80000))
 (segment (start 210.312 121.92) (end 210.312 126.238) (width 0.5) (layer F.Cu) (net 8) (status 80000))
 (via (at 210.312 126.238) (size 0.889) (layers F.Cu B.Cu) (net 8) (status 80000))
 (segment (start 210.312 126.238) (end 210.312 128.016) (width 0.5) (layer B.Cu) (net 8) (status 80000))
 (segment (start 210.312 128.016) (end 211.836 129.54) (width 0.5) (layer B.Cu) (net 8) (status 80000))
 (segment (start 211.836 129.54) (end 212.344 129.54) (width 0.5) (layer B.Cu) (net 8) (status 80000))
 (segment (start 212.344 129.54) (end 212.348 129.418) (width 0.5) (layer B.Cu) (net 8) (status 80000))
 (segment (start 212.348 131.418) (end 212.344 131.318) (width 0.5) (layer B.Cu) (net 9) (status 80000))
 (segment (start 212.344 131.318) (end 211.836 130.81) (width 0.5) (layer B.Cu) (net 9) (status 80000))
 (segment (start 211.836 130.81) (end 211.074 130.81) (width 0.5) (layer B.Cu) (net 9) (status 80000))
 (segment (start 211.074 130.81) (end 209.804 129.54) (width 0.5) (layer B.Cu) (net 9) (status 80000))
 (segment (start 209.804 129.54) (end 209.55 129.54) (width 0.5) (layer B.Cu) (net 9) (status 80000))
 (via (at 209.55 129.54) (size 0.889) (layers F.Cu B.Cu) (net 9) (status 80000))
 (segment (start 209.55 129.54) (end 208.788 128.778) (width 0.5) (layer F.Cu) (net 9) (status 80000))
 (segment (start 208.788 128.778) (end 208.788 124.968) (width 0.5) (layer F.Cu) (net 9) (status 80000))
 (segment (start 208.788 124.968) (end 207.518 123.698) (width 0.5) (layer F.Cu) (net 9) (status 80000))
 (segment (start 207.518 123.698) (end 207.518 121.666) (width 0.5) (layer F.Cu) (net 9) (status 80000))
 (segment (start 212.09 166.37) (end 212.09 163.576) (width 0.5) (layer F.Cu) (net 10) (status 80000))
 (via (at 212.09 163.576) (size 0.889) (layers F.Cu B.Cu) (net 10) (status 80000))
 (segment (start 212.09 163.576) (end 209.804 161.29) (width 0.5) (layer B.Cu) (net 10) (status 80000))
 (via (at 209.804 161.29) (size 0.889) (layers F.Cu B.Cu) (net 10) (status 80000))
 (segment (start 209.804 161.29) (end 209.296 160.782) (width 0.5) (layer F.Cu) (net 10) (status 80000))
 (segment (start 209.296 160.782) (end 209.296 135.382) (width 0.5) (layer F.Cu) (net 10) (status 80000))
 (segment (start 209.296 135.382) (end 208.28 134.366) (width 0.5) (layer F.Cu) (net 10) (status 80000))
 (segment (start 208.28 134.366) (end 208.28 133.35) (width 0.5) (layer F.Cu) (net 10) (status 80000))
 (segment (start 208.28 133.35) (end 207.264 132.334) (width 0.5) (layer F.Cu) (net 10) (status 80000))
 (segment (start 207.264 132.334) (end 207.264 130.302) (width 0.5) (layer F.Cu) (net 10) (status 80000))
 (segment (start 207.264 130.302) (end 207.01 130.048) (width 0.5) (layer F.Cu) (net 10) (status 80000))
 (segment (start 207.01 130.048) (end 207.01 129.032) (width 0.5) (layer F.Cu) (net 10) (status 80000))
 (via (at 207.01 129.032) (size 0.889) (layers F.Cu B.Cu) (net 10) (status 80000))
 (segment (start 207.01 129.032) (end 207.01 127.254) (width 0.5) (layer B.Cu) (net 10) (status 80000))
 (segment (start 207.01 127.254) (end 203.2 123.444) (width 0.5) (layer B.Cu) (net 10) (status 80000))
 (segment (start 203.2 123.444) (end 203.2 122.428) (width 0.5) (layer B.Cu) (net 10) (status 80000))
 (segment (start 203.2 122.428) (end 202.438 121.666) (width 0.5) (layer B.Cu) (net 10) (status 80000))
 (segment (start 168.656 125.222) (end 170.434 125.222) (width 0.5) (layer F.Cu) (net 11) (status 80000))
 (segment (start 170.434 125.222) (end 172.466 127.254) (width 0.5) (layer F.Cu) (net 11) (status 80000))
 (segment (start 172.466 127.254) (end 172.466 149.098) (width 0.5) (layer F.Cu) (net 11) (status 80000))
 (segment (start 172.466 149.098) (end 169.672 151.892) (width 0.5) (layer F.Cu) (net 11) (status 80000))
 (segment (start 169.672 151.892) (end 169.672 152.146) (width 0.5) (layer F.Cu) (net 11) (status 80000))
 (segment (start 179.832 120.65) (end 176.53 123.952) (width 0.5) (layer F.Cu) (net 11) (status 80000))
 (via (at 176.53 123.952) (size 0.889) (layers F.Cu B.Cu) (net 11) (status 80000))
 (segment (start 176.53 123.952) (end 175.26 125.222) (width 0.5) (layer B.Cu) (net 11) (status 80000))
 (segment (start 175.26 125.222) (end 168.656 125.222) (width 0.5) (layer B.Cu) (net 11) (status 80000))
 (segment (start 185.42 120.65) (end 179.832 120.65) (width 0.5) (layer B.Cu) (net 11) (status 80000))
 (segment (start 169.672 147.146) (end 169.672 147.066) (width 0.5) (layer F.Cu) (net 12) (status 80000))
 (segment (start 169.672 147.066) (end 166.37 150.368) (width 0.5) (layer F.Cu) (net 12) (status 80000))
 (segment (start 166.37 150.368) (end 166.37 156.21) (width 0.5) (layer F.Cu) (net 12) (status 80000))
 (segment (start 169.672 147.146) (end 169.672 142.146) (width 0.5) (layer F.Cu) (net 12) (status 80000))
 (segment (start 168.656 122.682) (end 168.91 122.428) (width 0.5) (layer B.Cu) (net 22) (status 80000))
 (segment (start 168.91 122.428) (end 186.436 122.428) (width 0.5) (layer B.Cu) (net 22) (status 80000))
 (segment (start 186.436 122.428) (end 188.214 120.65) (width 0.5) (layer B.Cu) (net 22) (status 80000))
 (segment (start 188.214 120.65) (end 190.754 120.65) (width 0.5) (layer B.Cu) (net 22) (status 80000))
 (segment (start 190.754 120.65) (end 196.088 120.65) (width 0.5) (layer B.Cu) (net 22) (status 80000))
 (segment (start 194.31 128.778) (end 193.294 129.794) (width 0.5) (layer F.Cu) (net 14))
 (segment (start 200.152 127.508) (end 200.66 127.508) (width 0.5) (layer B.Cu) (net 14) (status 80000))
 (segment (start 201.422 126.746) (end 200.66 127.508) (width 0.5) (layer B.Cu) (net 14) (status 80000))
 (segment (start 201.422 123.952) (end 201.422 126.746) (width 0.5) (layer B.Cu) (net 14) (status 80000))
 (segment (start 198.882 123.952) (end 201.422 123.952) (width 0.5) (layer B.Cu) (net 14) (status 80000))
 (segment (start 198.882 124.206) (end 198.882 123.952) (width 0.5) (layer B.Cu) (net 14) (status 80000))
 (segment (start 194.31 128.778) (end 198.882 124.206) (width 0.5) (layer B.Cu) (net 14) (status 80000))
 (via (at 194.31 128.778) (size 0.889) (layers F.Cu B.Cu) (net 14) (status 80000))
 (segment (start 188.976 141.224) (end 188.976 137.668) (width 0.5) (layer F.Cu) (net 14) (status 80000))
 (segment (start 188.468 141.732) (end 188.976 141.224) (width 0.5) (layer F.Cu) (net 14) (status 80000))
 (via (at 188.468 141.732) (size 0.889) (layers F.Cu B.Cu) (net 14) (status 80000))
 (segment (start 191.516 144.78) (end 188.468 141.732) (width 0.5) (layer B.Cu) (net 14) (status 80000))
 (via (at 191.516 144.78) (size 0.889) (layers F.Cu B.Cu) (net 14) (status 80000))
 (segment (start 191.516 152.654) (end 191.516 144.78) (width 0.5) (layer F.Cu) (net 14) (status 80000))
 (segment (start 194.056 155.194) (end 191.516 152.654) (width 0.5) (layer F.Cu) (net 14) (status 80000))
 (via (at 194.056 155.194) (size 0.889) (layers F.Cu B.Cu) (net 14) (status 80000))
 (segment (start 194.31 155.448) (end 194.056 155.194) (width 0.5) (layer B.Cu) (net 14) (status 80000))
 (segment (start 194.818 155.448) (end 194.31 155.448) (width 0.5) (layer B.Cu) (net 14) (status 80000))
 (segment (start 202.692 163.322) (end 194.818 155.448) (width 0.5) (layer B.Cu) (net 14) (status 80000))
 (segment (start 202.692 163.322) (end 202.692 165.608) (width 0.5) (layer B.Cu) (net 14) (status 80000))
 (segment (start 188.976 135.636) (end 188.976 137.668) (width 0.5) (layer F.Cu) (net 14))
 (segment (start 193.294 131.318) (end 188.976 135.636) (width 0.5) (layer F.Cu) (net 14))
 (segment (start 193.294 129.794) (end 193.294 131.318) (width 0.5) (layer F.Cu) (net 14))
 (segment (start 202.656 165.608) (end 202.692 165.608) (width 0.5) (layer B.Cu) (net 14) (status 80000))
 (segment (start 200.152 127.508) (end 200.148 127.418) (width 0.5) (layer B.Cu) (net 14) (status 80000))
 (segment (start 200.148 131.418) (end 200.152 131.318) (width 0.5) (layer B.Cu) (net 15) (status 80000))
 (segment (start 200.152 131.318) (end 200.406 131.064) (width 0.5) (layer B.Cu) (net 15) (status 80000))
 (segment (start 200.406 131.064) (end 201.93 131.064) (width 0.5) (layer B.Cu) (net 15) (status 80000))
 (via (at 201.93 131.064) (size 0.889) (layers F.Cu B.Cu) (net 15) (status 80000))
 (segment (start 201.93 131.064) (end 200.152 132.842) (width 0.5) (layer F.Cu) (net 15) (status 80000))
 (segment (start 200.152 132.842) (end 200.152 139.954) (width 0.5) (layer F.Cu) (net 15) (status 80000))
 (segment (start 200.152 139.954) (end 202.184 141.986) (width 0.5) (layer F.Cu) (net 15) (status 80000))
 (segment (start 202.184 141.986) (end 202.184 164.338) (width 0.5) (layer F.Cu) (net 15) (status 80000))
 (segment (start 202.184 164.338) (end 200.66 165.862) (width 0.5) (layer F.Cu) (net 15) (status 80000))
 (segment (start 200.66 165.862) (end 200.66 167.64) (width 0.5) (layer F.Cu) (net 15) (status 80000))
 (via (at 200.66 167.64) (size 0.889) (layers F.Cu B.Cu) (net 15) (status 80000))
 (segment (start 200.66 167.64) (end 200.152 167.132) (width 0.5) (layer B.Cu) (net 15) (status 80000))
 (segment (start 200.152 167.132) (end 200.152 165.608) (width 0.5) (layer B.Cu) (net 15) (status 80000))
 (segment (start 200.152 165.608) (end 200.126 165.608) (width 0.5) (layer B.Cu) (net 15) (status 80000))
 (segment (start 195.58 134.62) (end 194.564 135.636) (width 0.5) (layer B.Cu) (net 16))
 (segment (start 198.882 165.608) (end 198.882 164.084) (width 0.5) (layer B.Cu) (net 16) (status 80000))
 (segment (start 198.374 163.576) (end 198.882 164.084) (width 0.5) (layer B.Cu) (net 16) (status 80000))
 (via (at 198.374 163.576) (size 0.889) (layers F.Cu B.Cu) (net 16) (status 80000))
 (segment (start 198.374 148.844) (end 198.374 163.576) (width 0.5) (layer F.Cu) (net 16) (status 80000))
 (segment (start 194.056 144.526) (end 198.374 148.844) (width 0.5) (layer F.Cu) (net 16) (status 80000))
 (segment (start 194.056 144.018) (end 194.056 144.526) (width 0.5) (layer F.Cu) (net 16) (status 80000))
 (segment (start 193.802 143.764) (end 194.056 144.018) (width 0.5) (layer F.Cu) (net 16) (status 80000))
 (segment (start 193.802 143.256) (end 193.802 143.764) (width 0.5) (layer F.Cu) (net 16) (status 80000))
 (segment (start 191.516 140.97) (end 193.802 143.256) (width 0.5) (layer F.Cu) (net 16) (status 80000))
 (via (at 191.516 140.97) (size 0.889) (layers F.Cu B.Cu) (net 16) (status 80000))
 (segment (start 198.374 134.62) (end 195.58 134.62) (width 0.5) (layer B.Cu) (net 16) (status 80000))
 (segment (start 198.882 134.112) (end 198.374 134.62) (width 0.5) (layer B.Cu) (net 16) (status 80000))
 (segment (start 199.39 134.112) (end 198.882 134.112) (width 0.5) (layer B.Cu) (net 16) (status 80000))
 (segment (start 199.39 134.112) (end 200.152 133.35) (width 0.5) (layer B.Cu) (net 16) (status 80000))
 (segment (start 188.722 138.176) (end 191.516 140.97) (width 0.5) (layer B.Cu) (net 16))
 (segment (start 188.722 136.398) (end 188.722 138.176) (width 0.5) (layer B.Cu) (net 16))
 (segment (start 189.484 135.636) (end 188.722 136.398) (width 0.5) (layer B.Cu) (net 16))
 (segment (start 194.564 135.636) (end 189.484 135.636) (width 0.5) (layer B.Cu) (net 16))
 (segment (start 200.148 133.418) (end 200.152 133.35) (width 0.5) (layer B.Cu) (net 16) (status 80000))
 (segment (start 198.882 165.608) (end 198.846 165.608) (width 0.5) (layer B.Cu) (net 16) (status 80000))
 (segment (start 200.148 135.418) (end 200.152 135.382) (width 0.5) (layer B.Cu) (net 17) (status 80000))
 (segment (start 200.152 135.382) (end 199.644 135.89) (width 0.5) (layer B.Cu) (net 17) (status 80000))
 (segment (start 199.644 135.89) (end 196.342 135.89) (width 0.5) (layer B.Cu) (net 17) (status 80000))
 (via (at 196.342 135.89) (size 0.889) (layers F.Cu B.Cu) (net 17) (status 80000))
 (segment (start 196.342 135.89) (end 194.818 137.414) (width 0.5) (layer F.Cu) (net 17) (status 80000))
 (segment (start 194.818 137.414) (end 194.818 143.51) (width 0.5) (layer F.Cu) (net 17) (status 80000))
 (segment (start 194.818 143.51) (end 200.914 149.606) (width 0.5) (layer F.Cu) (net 17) (status 80000))
 (segment (start 200.914 149.606) (end 200.914 163.576) (width 0.5) (layer F.Cu) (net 17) (status 80000))
 (via (at 200.914 163.576) (size 0.889) (layers F.Cu B.Cu) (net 17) (status 80000))
 (segment (start 200.914 163.576) (end 201.422 164.084) (width 0.5) (layer B.Cu) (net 17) (status 80000))
 (segment (start 201.422 164.084) (end 201.422 165.608) (width 0.5) (layer B.Cu) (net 17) (status 80000))
 (segment (start 201.422 165.608) (end 201.396 165.608) (width 0.5) (layer B.Cu) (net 17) (status 80000)))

